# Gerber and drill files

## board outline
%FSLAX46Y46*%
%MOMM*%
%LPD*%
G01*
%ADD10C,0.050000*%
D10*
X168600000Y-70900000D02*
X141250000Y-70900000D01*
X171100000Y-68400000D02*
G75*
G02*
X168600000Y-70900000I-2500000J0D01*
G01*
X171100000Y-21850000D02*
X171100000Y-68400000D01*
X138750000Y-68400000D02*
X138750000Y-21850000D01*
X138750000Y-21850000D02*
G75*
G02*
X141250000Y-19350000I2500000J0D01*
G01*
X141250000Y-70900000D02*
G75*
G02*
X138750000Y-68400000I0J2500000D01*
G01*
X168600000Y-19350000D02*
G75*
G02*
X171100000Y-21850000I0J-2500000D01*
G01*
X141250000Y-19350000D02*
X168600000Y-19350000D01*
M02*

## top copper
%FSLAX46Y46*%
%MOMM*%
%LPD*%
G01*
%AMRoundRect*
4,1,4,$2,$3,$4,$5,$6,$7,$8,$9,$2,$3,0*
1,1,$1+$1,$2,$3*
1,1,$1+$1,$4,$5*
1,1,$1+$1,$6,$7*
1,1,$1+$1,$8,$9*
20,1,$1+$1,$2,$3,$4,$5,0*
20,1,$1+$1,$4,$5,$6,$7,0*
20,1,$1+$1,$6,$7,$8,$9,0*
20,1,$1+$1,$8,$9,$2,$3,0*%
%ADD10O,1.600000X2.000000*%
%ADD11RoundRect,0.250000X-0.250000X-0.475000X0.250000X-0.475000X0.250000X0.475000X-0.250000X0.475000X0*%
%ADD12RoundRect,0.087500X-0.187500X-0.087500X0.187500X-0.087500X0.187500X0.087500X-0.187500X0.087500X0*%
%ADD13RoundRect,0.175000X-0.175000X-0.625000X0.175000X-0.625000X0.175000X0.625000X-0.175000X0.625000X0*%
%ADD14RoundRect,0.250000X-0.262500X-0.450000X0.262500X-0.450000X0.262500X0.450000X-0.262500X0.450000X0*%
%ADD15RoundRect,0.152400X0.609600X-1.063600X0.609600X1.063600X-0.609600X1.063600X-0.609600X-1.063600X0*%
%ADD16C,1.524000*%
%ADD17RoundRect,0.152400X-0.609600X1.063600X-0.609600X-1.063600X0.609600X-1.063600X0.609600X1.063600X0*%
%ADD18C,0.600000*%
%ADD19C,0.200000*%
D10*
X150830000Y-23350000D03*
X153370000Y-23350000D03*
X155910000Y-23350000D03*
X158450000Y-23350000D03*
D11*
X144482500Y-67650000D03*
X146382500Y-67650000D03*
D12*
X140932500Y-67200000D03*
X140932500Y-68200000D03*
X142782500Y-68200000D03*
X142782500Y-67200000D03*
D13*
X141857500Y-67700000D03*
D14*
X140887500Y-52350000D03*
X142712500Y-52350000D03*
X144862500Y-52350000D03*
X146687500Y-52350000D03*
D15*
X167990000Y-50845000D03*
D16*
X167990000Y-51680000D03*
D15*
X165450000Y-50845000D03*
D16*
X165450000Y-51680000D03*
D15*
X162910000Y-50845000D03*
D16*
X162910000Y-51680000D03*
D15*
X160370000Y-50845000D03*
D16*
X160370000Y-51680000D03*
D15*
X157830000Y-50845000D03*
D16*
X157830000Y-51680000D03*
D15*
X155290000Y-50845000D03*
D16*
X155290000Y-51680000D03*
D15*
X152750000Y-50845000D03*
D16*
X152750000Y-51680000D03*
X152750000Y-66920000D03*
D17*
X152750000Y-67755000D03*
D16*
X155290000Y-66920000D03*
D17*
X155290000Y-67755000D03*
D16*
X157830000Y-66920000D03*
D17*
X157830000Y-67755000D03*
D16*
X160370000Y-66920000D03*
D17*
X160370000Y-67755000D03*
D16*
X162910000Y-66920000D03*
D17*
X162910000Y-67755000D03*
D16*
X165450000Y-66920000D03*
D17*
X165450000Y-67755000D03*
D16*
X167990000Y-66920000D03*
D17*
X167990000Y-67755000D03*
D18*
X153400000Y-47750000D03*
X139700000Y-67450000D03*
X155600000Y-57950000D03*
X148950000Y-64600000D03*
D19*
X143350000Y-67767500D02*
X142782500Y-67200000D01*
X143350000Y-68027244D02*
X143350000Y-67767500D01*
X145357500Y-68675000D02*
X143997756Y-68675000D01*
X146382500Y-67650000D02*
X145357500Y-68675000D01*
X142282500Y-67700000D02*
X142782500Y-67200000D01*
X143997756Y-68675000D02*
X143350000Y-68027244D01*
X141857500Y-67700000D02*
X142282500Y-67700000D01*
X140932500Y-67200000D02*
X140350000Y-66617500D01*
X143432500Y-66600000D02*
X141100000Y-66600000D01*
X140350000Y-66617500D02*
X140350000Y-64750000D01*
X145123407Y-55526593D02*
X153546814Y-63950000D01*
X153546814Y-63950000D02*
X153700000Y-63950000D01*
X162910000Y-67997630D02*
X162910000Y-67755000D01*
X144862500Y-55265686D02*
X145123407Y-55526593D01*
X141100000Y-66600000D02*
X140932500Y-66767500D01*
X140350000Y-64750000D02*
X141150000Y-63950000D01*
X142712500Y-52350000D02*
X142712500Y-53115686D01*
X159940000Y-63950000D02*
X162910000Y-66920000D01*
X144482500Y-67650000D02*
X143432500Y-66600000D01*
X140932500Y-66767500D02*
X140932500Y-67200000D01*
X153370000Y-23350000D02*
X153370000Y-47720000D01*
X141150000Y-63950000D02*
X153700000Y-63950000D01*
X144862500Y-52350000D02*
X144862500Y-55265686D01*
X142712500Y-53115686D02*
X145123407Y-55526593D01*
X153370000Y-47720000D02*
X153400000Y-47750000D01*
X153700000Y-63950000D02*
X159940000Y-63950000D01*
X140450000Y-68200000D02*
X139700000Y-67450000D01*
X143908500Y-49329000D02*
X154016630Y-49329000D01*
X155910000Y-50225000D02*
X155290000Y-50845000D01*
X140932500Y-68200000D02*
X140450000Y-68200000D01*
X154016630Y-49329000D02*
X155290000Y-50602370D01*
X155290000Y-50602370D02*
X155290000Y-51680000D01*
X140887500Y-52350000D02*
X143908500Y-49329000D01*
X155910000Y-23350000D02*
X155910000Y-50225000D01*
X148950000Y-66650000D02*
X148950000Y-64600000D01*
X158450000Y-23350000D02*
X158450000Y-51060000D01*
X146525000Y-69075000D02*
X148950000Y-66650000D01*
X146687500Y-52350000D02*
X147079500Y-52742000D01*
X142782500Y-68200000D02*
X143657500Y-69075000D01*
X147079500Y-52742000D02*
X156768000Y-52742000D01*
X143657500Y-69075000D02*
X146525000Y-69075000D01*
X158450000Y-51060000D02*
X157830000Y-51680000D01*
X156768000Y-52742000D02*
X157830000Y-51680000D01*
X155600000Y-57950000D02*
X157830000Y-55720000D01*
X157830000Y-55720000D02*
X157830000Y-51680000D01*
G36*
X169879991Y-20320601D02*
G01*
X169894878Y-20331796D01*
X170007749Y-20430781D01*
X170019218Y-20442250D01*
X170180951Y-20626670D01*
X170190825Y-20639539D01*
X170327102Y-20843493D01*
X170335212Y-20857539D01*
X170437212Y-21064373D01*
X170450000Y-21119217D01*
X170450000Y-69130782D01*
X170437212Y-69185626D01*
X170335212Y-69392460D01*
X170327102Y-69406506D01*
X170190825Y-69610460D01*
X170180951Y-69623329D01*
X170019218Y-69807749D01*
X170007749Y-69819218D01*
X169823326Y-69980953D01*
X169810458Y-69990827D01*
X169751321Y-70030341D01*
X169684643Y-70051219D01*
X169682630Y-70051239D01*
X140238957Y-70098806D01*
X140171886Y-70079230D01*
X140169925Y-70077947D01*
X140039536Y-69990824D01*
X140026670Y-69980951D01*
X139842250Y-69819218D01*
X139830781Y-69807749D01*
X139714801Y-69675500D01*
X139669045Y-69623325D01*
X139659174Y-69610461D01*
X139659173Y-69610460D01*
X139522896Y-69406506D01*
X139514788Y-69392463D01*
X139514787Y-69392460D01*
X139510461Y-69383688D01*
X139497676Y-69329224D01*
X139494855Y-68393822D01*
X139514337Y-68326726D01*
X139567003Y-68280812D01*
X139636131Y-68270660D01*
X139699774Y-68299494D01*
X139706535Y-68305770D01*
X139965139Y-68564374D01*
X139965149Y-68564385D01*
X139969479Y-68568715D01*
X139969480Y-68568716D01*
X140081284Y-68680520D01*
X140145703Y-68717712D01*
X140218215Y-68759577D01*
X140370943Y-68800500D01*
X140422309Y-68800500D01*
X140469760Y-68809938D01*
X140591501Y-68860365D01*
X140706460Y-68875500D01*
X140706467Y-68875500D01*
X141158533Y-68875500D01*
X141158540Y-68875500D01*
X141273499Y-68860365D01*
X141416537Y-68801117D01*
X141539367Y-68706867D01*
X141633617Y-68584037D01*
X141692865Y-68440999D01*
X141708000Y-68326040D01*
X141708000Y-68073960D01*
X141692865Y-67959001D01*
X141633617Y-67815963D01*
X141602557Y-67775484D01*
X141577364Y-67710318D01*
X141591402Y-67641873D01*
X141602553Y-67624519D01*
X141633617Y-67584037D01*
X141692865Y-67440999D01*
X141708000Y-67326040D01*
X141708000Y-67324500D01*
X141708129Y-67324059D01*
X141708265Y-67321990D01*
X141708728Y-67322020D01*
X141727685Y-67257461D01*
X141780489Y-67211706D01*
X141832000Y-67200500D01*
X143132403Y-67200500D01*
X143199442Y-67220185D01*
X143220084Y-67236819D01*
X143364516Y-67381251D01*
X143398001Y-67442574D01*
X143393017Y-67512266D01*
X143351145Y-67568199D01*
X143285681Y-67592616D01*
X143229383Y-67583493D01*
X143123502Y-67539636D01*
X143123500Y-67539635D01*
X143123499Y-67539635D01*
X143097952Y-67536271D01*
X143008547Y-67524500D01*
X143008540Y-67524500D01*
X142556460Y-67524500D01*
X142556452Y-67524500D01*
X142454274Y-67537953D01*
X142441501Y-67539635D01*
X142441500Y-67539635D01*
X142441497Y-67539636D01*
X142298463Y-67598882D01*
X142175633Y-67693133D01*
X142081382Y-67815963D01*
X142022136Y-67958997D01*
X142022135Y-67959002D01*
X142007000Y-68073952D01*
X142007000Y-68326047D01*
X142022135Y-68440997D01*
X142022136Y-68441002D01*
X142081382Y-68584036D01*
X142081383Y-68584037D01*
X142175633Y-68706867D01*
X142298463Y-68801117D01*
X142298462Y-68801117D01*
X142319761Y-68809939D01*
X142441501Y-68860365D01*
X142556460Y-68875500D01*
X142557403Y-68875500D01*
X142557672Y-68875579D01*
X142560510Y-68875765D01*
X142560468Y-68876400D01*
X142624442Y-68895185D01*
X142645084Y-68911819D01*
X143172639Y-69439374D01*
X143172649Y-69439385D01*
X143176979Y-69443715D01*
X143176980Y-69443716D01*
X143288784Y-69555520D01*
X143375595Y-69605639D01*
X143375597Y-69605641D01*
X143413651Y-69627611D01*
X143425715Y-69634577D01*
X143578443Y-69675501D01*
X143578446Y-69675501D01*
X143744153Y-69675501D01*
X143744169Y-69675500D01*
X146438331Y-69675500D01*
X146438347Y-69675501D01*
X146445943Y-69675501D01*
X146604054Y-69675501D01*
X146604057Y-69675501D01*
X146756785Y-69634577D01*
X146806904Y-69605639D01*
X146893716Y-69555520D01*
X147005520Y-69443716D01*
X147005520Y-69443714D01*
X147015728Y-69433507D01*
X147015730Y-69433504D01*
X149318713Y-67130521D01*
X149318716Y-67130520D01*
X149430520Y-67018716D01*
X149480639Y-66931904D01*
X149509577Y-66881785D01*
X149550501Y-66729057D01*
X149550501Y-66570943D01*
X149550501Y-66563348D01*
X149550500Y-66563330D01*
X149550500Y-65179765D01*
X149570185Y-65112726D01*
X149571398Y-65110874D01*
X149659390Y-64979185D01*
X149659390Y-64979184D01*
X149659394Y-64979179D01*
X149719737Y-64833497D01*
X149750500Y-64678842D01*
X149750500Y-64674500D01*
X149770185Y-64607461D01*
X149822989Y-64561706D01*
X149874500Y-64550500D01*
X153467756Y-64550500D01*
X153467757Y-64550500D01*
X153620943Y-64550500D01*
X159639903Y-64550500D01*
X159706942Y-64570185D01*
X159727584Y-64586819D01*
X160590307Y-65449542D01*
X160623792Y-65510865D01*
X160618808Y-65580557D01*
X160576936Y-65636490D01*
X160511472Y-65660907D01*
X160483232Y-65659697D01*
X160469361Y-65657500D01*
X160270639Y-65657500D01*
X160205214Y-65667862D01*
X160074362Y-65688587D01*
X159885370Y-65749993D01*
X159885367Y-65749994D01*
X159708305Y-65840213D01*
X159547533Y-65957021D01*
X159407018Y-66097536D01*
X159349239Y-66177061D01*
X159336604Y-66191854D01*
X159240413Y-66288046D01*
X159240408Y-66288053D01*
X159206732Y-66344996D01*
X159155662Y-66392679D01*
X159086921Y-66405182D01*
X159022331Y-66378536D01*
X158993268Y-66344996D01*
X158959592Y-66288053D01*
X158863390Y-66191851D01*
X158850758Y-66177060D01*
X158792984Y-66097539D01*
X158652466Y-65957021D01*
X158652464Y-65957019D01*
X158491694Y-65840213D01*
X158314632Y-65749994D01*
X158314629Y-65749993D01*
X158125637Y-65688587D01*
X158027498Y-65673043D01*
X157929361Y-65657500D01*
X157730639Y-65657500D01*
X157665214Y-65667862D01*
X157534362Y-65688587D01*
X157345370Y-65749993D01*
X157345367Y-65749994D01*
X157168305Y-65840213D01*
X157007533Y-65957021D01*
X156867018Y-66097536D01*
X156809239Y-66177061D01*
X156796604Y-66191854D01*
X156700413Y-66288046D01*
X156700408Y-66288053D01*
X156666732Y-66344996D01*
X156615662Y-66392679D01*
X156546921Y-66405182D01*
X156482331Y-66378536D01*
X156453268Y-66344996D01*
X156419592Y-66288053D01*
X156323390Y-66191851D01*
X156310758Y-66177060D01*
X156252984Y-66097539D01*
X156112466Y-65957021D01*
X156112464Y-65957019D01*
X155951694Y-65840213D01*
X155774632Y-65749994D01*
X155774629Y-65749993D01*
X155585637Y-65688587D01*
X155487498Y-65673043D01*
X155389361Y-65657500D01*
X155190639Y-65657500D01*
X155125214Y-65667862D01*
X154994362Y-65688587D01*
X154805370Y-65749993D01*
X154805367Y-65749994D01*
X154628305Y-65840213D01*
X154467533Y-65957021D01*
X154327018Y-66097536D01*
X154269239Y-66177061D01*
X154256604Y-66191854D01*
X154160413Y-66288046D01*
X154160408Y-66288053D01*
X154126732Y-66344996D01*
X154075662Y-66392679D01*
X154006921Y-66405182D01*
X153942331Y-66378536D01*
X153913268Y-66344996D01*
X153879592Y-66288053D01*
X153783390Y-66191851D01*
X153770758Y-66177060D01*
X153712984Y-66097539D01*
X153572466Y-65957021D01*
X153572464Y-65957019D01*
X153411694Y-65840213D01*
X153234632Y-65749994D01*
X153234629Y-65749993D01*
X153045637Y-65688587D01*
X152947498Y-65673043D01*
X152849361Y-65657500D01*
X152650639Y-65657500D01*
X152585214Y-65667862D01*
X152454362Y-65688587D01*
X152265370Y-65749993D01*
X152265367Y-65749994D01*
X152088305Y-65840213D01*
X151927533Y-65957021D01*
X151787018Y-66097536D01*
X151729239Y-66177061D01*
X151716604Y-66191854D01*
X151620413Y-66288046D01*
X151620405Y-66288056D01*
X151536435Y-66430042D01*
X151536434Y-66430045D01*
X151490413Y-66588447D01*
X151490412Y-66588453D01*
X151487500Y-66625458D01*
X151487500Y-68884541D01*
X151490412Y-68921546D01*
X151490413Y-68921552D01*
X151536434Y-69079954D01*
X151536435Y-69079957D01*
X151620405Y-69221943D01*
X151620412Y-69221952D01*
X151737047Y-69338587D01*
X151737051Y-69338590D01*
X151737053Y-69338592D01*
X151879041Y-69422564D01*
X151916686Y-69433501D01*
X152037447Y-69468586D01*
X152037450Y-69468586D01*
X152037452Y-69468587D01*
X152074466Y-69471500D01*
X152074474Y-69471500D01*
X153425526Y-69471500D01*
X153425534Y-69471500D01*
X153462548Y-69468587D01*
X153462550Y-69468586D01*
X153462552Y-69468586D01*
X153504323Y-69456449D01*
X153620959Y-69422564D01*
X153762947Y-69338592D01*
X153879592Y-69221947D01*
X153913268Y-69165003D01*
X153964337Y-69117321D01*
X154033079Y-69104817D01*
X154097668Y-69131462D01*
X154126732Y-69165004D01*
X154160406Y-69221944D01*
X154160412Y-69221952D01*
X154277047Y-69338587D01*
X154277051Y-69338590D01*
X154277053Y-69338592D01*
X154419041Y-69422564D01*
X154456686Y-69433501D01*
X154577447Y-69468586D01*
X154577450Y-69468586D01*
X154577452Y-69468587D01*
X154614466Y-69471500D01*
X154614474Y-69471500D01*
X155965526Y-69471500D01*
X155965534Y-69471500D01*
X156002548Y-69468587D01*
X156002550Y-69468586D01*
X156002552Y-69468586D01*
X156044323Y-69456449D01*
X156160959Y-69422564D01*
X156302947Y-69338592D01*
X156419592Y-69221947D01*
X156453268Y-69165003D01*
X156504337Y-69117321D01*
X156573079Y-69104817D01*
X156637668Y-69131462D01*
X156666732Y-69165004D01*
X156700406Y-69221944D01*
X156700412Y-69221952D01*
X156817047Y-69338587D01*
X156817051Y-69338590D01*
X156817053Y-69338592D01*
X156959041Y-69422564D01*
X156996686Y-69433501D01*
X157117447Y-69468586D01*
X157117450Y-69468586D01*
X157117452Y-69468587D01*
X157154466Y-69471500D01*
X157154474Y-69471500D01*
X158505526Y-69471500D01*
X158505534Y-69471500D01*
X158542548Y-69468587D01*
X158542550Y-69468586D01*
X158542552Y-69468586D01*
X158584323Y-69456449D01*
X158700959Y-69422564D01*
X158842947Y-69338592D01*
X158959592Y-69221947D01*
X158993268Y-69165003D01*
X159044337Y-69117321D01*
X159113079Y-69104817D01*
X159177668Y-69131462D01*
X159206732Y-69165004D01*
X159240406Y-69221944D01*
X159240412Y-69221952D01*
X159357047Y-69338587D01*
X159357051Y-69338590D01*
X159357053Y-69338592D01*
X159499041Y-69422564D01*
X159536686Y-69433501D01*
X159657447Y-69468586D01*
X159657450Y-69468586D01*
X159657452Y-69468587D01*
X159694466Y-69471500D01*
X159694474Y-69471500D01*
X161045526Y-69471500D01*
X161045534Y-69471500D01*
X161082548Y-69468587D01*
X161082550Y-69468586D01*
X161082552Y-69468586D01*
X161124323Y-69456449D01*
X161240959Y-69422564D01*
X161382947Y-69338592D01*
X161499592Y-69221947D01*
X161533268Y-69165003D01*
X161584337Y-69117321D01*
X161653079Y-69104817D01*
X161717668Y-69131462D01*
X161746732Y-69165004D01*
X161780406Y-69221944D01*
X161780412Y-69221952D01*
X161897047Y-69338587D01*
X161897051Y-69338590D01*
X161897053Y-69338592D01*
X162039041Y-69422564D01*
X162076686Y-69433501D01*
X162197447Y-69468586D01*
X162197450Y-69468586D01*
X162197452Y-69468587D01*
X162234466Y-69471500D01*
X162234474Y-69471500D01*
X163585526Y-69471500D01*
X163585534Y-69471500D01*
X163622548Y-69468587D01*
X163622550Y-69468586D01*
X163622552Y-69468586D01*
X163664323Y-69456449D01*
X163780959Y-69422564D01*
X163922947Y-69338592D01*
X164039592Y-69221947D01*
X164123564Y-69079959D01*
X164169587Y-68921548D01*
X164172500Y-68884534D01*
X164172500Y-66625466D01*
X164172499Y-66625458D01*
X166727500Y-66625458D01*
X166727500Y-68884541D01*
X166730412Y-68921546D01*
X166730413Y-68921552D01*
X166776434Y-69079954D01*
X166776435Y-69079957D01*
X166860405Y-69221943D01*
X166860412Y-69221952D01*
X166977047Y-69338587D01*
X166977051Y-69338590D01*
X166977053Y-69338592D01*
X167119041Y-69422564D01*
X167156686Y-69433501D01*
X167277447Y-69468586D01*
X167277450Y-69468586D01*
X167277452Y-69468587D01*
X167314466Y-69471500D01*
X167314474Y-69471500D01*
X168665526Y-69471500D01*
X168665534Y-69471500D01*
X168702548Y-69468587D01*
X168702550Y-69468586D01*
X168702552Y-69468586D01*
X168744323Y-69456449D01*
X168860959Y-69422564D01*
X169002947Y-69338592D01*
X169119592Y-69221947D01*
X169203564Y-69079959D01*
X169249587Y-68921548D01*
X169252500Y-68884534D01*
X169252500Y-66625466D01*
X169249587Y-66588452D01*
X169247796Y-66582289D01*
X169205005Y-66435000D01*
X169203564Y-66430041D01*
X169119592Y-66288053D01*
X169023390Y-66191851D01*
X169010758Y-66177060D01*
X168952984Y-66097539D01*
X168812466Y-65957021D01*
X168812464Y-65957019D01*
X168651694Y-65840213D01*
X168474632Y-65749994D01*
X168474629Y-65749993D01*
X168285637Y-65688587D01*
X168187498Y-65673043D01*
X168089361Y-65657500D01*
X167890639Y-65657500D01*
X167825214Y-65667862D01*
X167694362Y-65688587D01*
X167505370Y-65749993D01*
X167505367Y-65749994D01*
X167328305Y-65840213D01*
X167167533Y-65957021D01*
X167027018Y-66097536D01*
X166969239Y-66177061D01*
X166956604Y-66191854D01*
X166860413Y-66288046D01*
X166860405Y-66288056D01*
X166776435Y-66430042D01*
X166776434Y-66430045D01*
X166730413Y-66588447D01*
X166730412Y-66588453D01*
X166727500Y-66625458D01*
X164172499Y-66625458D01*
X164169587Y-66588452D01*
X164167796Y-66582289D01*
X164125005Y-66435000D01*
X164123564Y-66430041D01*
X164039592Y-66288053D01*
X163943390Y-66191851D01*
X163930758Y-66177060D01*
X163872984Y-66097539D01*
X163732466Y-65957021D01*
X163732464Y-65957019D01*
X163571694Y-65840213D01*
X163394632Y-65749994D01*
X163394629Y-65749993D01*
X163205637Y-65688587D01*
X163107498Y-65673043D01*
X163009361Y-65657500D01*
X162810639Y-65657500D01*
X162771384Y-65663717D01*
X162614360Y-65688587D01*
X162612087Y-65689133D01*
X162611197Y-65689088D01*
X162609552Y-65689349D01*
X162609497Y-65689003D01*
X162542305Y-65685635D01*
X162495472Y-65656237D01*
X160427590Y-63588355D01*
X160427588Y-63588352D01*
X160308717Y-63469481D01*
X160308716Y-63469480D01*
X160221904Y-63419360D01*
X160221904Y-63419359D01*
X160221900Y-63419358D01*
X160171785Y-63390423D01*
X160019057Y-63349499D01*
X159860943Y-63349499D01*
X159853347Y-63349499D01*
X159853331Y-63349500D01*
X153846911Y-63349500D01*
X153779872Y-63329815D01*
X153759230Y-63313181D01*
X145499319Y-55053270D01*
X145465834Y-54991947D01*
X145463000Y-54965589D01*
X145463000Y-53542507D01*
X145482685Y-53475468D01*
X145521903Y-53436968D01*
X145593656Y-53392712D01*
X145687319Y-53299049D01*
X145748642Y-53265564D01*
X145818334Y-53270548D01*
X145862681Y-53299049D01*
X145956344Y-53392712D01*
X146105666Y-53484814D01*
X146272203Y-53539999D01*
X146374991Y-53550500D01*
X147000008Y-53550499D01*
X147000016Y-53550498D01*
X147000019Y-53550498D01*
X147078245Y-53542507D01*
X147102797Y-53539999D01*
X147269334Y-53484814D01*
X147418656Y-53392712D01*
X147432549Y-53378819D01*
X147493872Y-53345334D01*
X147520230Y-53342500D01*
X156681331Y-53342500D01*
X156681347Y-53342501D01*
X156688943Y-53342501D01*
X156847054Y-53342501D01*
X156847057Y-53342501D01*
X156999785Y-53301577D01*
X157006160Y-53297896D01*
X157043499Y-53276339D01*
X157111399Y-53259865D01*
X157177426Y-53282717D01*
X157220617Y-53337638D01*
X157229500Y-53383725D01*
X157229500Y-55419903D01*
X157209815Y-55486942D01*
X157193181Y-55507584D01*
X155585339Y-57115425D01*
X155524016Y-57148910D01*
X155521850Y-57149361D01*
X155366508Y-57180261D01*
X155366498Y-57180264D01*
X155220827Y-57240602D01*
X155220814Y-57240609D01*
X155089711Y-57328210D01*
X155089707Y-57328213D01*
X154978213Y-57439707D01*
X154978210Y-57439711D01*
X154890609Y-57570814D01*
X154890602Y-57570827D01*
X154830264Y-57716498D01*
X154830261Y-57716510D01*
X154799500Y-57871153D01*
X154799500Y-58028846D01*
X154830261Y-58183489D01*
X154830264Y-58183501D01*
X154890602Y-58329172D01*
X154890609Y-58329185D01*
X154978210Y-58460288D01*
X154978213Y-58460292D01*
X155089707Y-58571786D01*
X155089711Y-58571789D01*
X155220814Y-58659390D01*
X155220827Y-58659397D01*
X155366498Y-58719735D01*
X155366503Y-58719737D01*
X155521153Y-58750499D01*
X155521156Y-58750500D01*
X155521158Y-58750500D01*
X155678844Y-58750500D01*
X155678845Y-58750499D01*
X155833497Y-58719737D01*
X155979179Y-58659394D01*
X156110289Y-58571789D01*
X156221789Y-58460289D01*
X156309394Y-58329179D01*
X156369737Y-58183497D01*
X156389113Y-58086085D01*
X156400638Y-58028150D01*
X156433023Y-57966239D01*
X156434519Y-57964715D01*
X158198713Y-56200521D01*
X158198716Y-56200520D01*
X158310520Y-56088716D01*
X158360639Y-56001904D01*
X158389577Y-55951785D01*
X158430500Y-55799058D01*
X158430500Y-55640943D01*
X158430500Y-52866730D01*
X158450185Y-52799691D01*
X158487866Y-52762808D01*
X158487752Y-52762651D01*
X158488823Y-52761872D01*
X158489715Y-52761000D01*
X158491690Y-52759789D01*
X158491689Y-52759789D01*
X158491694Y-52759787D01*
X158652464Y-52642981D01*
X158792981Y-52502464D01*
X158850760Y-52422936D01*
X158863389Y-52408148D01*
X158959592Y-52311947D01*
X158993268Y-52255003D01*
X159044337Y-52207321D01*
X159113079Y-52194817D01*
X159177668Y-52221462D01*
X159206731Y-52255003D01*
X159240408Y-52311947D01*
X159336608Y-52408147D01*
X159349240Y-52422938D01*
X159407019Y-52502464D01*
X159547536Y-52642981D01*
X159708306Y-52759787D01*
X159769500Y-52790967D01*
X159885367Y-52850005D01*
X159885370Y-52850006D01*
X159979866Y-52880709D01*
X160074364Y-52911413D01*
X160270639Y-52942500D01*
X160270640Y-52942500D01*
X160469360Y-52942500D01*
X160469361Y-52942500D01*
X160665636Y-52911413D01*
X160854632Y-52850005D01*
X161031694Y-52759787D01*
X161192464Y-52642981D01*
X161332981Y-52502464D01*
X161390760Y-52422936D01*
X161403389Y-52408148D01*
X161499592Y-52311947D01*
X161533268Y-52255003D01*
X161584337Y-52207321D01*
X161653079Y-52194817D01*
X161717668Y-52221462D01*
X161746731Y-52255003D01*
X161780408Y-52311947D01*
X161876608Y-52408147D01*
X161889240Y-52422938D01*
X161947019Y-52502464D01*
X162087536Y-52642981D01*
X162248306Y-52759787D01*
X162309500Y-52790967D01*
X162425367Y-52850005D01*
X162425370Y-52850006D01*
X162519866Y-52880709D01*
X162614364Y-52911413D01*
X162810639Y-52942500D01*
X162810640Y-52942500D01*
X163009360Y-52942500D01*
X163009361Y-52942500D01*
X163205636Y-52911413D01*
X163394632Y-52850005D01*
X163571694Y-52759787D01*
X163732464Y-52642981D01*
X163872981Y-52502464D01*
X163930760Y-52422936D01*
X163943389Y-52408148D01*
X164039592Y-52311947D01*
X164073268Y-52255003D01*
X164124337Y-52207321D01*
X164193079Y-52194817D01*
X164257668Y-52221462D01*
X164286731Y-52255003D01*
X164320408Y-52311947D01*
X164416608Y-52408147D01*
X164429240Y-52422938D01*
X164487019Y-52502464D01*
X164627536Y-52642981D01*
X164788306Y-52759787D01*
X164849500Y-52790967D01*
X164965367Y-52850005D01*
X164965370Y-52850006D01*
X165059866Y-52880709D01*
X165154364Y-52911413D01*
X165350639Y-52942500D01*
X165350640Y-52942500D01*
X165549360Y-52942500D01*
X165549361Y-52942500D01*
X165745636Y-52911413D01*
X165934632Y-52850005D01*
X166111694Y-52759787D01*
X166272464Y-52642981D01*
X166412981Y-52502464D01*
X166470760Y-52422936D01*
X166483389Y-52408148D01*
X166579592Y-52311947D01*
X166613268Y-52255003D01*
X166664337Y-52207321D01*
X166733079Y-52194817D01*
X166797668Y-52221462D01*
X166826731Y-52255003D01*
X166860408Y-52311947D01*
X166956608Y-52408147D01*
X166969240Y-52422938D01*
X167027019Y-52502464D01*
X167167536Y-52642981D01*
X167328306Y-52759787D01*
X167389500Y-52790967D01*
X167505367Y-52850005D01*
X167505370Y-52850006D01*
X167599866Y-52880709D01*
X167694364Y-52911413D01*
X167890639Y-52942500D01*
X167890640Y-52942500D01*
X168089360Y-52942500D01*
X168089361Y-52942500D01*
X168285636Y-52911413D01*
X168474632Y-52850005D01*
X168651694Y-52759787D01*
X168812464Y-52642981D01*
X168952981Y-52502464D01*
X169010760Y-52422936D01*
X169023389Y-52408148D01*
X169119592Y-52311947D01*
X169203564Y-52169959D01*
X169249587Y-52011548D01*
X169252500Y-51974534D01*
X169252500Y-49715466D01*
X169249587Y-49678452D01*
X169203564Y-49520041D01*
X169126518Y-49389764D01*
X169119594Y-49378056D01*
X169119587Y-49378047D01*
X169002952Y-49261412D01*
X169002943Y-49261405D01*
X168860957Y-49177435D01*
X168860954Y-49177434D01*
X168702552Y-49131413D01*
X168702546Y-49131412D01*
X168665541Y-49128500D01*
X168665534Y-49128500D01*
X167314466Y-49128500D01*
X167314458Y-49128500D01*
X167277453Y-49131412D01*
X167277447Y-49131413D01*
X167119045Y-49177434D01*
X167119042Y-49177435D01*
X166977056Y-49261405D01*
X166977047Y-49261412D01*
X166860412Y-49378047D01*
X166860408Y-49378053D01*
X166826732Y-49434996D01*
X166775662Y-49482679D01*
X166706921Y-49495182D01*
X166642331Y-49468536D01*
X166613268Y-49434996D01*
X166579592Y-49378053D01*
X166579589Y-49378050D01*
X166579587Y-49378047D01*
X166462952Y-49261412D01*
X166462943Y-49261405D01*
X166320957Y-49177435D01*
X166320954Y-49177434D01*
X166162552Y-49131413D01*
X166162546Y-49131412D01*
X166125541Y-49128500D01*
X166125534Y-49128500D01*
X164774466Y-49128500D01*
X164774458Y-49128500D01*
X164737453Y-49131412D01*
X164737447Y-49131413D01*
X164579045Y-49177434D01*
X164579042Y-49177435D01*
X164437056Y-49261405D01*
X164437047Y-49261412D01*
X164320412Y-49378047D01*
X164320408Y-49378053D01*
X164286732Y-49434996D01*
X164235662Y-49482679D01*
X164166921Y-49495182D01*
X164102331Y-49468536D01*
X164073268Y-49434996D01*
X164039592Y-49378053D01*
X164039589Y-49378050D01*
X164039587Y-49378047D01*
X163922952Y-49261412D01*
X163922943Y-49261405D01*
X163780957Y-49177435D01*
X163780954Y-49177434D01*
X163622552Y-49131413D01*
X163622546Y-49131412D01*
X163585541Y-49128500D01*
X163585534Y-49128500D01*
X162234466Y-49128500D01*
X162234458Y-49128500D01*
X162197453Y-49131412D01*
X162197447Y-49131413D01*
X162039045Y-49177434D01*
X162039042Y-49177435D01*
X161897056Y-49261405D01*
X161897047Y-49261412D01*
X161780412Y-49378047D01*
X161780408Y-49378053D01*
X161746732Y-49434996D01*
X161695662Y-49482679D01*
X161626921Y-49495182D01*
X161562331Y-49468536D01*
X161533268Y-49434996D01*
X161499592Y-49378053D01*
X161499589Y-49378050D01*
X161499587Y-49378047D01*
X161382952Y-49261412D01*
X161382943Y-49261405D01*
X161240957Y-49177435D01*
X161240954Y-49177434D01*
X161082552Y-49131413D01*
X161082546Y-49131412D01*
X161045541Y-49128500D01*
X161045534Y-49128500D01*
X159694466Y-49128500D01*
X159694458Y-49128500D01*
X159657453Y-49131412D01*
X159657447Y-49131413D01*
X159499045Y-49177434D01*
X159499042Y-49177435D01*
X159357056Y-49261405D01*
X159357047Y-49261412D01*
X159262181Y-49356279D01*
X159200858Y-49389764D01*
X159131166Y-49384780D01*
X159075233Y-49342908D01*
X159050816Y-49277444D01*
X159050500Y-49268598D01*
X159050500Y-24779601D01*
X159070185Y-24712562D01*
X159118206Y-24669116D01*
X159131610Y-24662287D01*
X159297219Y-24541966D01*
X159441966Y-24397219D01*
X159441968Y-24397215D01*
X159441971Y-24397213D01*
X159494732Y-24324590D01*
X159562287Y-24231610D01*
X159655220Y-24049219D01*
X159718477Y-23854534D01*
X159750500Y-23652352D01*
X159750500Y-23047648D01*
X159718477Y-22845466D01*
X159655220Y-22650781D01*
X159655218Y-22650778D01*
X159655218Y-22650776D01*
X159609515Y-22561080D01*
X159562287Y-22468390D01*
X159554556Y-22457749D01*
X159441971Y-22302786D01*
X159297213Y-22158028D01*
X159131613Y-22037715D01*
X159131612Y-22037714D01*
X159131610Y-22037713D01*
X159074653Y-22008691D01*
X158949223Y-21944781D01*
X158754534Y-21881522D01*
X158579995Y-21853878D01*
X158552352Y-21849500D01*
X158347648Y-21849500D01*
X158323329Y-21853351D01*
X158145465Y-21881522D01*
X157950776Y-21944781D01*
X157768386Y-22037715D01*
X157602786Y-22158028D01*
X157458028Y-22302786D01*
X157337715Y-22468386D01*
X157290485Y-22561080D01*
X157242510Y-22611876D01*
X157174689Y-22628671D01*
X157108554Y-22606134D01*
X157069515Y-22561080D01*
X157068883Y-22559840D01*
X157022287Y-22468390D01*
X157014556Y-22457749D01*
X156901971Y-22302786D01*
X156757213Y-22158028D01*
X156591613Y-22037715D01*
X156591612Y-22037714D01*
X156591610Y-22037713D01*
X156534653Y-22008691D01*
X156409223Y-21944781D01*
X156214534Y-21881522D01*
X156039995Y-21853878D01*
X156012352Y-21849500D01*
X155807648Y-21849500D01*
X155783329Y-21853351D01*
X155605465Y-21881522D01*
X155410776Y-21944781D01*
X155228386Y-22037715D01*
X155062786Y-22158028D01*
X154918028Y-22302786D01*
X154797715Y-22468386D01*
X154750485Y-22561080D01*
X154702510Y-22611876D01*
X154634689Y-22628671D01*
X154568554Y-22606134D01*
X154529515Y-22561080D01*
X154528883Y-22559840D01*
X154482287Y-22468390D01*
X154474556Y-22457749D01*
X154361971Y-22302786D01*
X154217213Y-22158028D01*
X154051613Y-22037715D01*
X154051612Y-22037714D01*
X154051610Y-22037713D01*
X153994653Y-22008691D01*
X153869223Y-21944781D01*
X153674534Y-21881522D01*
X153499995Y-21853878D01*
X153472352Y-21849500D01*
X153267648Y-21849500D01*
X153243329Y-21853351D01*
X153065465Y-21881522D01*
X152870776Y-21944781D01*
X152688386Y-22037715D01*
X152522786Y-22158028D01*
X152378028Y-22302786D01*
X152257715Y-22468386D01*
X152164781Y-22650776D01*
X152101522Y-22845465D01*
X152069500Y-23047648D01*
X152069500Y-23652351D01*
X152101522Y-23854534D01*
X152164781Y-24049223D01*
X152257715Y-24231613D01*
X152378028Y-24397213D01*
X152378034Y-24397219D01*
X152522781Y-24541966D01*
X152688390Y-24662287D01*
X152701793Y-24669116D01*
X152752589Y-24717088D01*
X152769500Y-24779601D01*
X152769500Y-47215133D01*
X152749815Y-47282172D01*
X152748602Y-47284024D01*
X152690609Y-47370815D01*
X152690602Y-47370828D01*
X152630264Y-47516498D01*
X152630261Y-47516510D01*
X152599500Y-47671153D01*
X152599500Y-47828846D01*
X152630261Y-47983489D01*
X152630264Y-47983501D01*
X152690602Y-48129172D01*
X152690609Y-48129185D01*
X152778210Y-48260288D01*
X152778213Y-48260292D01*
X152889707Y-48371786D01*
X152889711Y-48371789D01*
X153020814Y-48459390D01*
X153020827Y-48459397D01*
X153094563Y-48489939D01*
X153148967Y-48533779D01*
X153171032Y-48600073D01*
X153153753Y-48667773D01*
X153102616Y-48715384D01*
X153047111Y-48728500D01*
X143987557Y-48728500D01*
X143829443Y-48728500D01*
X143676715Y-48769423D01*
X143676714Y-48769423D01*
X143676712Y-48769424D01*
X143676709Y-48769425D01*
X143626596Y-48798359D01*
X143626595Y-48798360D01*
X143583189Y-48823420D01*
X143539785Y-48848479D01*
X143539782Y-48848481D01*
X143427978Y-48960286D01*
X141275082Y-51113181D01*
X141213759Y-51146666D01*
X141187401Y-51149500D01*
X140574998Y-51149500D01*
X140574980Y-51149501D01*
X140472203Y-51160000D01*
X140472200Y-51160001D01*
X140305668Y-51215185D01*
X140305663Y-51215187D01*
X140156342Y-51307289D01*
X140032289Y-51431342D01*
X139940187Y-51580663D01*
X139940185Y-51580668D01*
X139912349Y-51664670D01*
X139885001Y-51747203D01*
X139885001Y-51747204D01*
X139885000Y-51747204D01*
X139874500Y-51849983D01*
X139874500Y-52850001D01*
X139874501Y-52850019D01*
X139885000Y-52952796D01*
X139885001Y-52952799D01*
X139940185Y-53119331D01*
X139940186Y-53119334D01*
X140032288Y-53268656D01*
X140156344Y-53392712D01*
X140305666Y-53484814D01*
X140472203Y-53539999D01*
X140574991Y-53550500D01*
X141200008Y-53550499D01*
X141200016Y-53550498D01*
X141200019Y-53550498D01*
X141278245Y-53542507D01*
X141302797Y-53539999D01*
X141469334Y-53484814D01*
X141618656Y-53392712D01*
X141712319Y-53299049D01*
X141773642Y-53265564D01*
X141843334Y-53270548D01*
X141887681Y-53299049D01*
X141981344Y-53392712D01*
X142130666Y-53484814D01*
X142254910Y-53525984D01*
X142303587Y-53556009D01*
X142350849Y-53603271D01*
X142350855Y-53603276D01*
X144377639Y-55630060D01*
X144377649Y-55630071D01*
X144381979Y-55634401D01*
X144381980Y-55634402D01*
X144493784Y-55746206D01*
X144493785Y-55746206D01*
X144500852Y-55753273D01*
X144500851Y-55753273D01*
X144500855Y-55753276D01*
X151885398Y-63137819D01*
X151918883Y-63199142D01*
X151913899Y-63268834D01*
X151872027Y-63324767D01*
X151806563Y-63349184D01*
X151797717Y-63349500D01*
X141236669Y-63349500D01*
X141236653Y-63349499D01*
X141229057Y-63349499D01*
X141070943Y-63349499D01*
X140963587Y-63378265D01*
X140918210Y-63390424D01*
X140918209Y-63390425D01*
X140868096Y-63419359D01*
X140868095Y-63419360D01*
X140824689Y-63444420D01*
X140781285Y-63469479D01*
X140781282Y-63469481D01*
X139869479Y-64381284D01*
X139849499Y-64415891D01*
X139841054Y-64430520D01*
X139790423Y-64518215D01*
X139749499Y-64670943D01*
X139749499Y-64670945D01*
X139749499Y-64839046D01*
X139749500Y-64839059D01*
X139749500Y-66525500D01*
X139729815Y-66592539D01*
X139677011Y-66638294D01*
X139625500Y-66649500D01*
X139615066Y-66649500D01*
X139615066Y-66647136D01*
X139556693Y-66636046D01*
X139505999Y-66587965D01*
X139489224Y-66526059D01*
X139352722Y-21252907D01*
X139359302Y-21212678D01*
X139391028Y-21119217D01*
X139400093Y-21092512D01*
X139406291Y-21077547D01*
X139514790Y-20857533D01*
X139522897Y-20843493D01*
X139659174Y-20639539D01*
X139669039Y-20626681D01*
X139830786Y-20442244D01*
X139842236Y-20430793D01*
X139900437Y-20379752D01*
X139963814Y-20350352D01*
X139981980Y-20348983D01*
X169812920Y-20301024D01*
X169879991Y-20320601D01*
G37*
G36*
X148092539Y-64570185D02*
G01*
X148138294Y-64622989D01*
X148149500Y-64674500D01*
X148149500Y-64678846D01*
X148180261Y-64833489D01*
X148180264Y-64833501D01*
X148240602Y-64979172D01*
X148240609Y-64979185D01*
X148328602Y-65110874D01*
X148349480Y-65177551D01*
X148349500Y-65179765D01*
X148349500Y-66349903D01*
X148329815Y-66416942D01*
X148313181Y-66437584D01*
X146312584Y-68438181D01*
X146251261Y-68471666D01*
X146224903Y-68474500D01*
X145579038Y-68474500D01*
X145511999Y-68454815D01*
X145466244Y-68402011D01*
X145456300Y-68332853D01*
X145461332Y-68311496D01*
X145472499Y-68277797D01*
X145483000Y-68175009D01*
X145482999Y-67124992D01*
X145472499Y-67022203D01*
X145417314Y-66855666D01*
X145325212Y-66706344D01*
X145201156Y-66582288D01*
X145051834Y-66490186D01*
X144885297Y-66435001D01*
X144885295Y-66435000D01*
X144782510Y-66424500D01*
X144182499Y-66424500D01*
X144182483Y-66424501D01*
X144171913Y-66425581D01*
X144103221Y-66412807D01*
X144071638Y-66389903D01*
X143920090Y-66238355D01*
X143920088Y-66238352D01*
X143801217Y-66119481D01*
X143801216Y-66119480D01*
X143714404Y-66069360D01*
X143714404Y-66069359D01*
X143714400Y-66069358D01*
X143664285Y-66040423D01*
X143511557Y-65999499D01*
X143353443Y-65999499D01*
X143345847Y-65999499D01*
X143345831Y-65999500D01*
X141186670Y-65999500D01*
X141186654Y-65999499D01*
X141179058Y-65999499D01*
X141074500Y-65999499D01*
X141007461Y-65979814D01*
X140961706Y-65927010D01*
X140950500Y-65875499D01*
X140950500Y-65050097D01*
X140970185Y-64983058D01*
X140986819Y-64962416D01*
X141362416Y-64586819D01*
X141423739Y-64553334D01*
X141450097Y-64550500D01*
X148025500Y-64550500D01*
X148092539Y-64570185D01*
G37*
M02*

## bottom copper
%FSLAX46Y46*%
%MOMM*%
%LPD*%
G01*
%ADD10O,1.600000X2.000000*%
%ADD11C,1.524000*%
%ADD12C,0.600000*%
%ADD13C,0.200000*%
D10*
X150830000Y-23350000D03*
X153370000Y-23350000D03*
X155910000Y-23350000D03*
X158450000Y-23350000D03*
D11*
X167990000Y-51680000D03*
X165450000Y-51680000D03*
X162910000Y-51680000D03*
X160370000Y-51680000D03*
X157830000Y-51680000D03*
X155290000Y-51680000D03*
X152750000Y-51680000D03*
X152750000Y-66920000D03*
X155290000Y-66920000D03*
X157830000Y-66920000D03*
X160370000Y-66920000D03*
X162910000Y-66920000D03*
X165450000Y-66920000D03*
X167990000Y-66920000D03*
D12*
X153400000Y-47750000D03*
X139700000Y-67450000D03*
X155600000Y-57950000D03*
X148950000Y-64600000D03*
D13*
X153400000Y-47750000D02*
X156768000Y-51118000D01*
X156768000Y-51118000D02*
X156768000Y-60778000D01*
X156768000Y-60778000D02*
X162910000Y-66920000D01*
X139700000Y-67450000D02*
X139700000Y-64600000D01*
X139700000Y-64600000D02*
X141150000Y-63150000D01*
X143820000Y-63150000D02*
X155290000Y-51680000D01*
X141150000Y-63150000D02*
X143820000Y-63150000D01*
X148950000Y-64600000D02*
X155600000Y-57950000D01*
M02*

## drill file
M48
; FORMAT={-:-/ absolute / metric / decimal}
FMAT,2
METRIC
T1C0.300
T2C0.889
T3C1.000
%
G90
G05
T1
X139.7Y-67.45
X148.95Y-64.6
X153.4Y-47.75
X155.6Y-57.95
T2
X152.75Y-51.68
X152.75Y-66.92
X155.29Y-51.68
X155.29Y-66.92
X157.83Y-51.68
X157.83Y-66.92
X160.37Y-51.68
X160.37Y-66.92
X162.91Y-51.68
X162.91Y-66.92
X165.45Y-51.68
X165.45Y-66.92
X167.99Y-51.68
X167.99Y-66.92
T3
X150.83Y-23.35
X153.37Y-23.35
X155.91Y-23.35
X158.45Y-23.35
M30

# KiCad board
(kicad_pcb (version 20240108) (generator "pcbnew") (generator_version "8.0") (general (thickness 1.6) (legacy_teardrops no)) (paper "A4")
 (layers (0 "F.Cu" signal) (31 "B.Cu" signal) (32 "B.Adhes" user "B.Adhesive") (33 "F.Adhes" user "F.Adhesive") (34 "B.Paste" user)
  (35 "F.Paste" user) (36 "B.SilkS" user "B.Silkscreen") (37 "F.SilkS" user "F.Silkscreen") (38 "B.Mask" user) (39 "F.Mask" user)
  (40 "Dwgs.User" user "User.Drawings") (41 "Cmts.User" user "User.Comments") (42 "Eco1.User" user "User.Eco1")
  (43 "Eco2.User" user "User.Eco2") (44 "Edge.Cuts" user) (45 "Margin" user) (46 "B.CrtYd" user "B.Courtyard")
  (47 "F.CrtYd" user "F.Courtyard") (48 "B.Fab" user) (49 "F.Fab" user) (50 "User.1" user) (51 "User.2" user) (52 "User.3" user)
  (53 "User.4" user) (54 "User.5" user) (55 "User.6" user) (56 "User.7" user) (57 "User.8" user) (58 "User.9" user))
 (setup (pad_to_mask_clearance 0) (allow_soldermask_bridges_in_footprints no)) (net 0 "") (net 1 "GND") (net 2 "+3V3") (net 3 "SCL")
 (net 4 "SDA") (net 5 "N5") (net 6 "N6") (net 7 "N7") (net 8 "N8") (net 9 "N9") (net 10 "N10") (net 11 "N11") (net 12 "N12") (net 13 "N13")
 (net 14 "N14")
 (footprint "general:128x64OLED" (layer "F.Cu") (at 154.45 33.95)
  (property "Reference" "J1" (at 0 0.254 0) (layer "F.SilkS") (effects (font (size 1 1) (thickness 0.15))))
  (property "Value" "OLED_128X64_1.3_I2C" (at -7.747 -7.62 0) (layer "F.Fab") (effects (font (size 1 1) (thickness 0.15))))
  (pad "1" thru_hole oval (at -3.62 -10.6 90) (size 2 1.6) (drill 1) (layers "*.Cu" "*.Mask") (remove_unused_layers no) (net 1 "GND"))
  (pad "2" thru_hole oval (at -1.08 -10.6 90) (size 2 1.6) (drill 1) (layers "*.Cu" "*.Mask") (remove_unused_layers no) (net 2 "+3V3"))
  (pad "3" thru_hole oval (at 1.46 -10.6 90) (size 2 1.6) (drill 1) (layers "*.Cu" "*.Mask") (remove_unused_layers no) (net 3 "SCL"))
  (pad "4" thru_hole oval (at 4 -10.6 90) (size 2 1.6) (drill 1) (layers "*.Cu" "*.Mask") (remove_unused_layers no) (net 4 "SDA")))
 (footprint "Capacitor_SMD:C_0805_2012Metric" (layer "F.Cu") (at 145.4325 67.65)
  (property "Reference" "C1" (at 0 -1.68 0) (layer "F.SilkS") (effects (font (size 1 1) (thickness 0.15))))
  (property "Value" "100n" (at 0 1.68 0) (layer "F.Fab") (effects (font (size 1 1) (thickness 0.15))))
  (pad "1" smd roundrect (at -0.95 0) (size 1 1.45) (layers "F.Cu" "F.Paste" "F.Mask") (roundrect_rratio 0.25) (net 2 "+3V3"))
  (pad "2" smd roundrect (at 0.95 0) (size 1 1.45) (layers "F.Cu" "F.Paste" "F.Mask") (roundrect_rratio 0.25) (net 1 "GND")))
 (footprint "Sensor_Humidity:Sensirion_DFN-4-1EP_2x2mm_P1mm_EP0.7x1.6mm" (layer "F.Cu") (at 141.8575 67.7)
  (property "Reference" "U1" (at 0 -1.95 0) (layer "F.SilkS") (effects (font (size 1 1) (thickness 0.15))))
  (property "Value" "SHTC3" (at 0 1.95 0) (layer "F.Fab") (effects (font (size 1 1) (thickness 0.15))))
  (pad "" smd roundrect (at -1.025 -0.5) (size 0.55 0.35) (layers "F.Paste") (roundrect_rratio 0.25))
  (pad "" smd roundrect (at -1.025 0.5) (size 0.55 0.35) (layers "F.Paste") (roundrect_rratio 0.25))
  (pad "" smd roundrect (at 0 0) (size 0.5 1.4) (layers "F.Paste") (roundrect_rratio 0.25))
  (pad "" smd roundrect (at 1.025 -0.5 180) (size 0.55 0.35) (layers "F.Paste") (roundrect_rratio 0.25))
  (pad "" smd roundrect (at 1.025 0.5 180) (size 0.55 0.35) (layers "F.Paste") (roundrect_rratio 0.25))
  (pad "1" smd roundrect (at -0.925 -0.5) (size 0.55 0.35) (layers "F.Cu" "F.Mask") (roundrect_rratio 0.25) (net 2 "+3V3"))
  (pad "2" smd roundrect (at -0.925 0.5) (size 0.55 0.35) (layers "F.Cu" "F.Mask") (roundrect_rratio 0.25) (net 3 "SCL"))
  (pad "3" smd roundrect (at 0.925 0.5) (size 0.55 0.35) (layers "F.Cu" "F.Mask") (roundrect_rratio 0.25) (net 4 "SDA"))
  (pad "4" smd roundrect (at 0.925 -0.5) (size 0.55 0.35) (layers "F.Cu" "F.Mask") (roundrect_rratio 0.25) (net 1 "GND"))
  (pad "5" smd roundrect (at 0 0) (size 0.7 1.6) (layers "F.Cu" "F.Mask") (roundrect_rratio 0.25) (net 1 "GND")))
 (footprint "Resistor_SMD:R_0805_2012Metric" (layer "F.Cu") (at 141.8 52.35)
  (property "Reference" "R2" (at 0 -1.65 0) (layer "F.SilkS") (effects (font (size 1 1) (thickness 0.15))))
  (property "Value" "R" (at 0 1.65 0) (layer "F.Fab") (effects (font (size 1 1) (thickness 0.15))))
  (pad "1" smd roundrect (at -0.9125 0) (size 1.025 1.4) (layers "F.Cu" "F.Paste" "F.Mask") (roundrect_rratio 0.243902) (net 3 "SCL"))
  (pad "2" smd roundrect (at 0.9125 0) (size 1.025 1.4) (layers "F.Cu" "F.Paste" "F.Mask") (roundrect_rratio 0.243902) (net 2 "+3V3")))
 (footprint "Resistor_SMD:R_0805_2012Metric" (layer "F.Cu") (at 145.775 52.35)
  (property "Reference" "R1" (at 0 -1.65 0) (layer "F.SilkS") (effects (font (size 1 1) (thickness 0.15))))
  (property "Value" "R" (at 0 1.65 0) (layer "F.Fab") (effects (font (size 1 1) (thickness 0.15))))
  (pad "1" smd roundrect (at -0.9125 0) (size 1.025 1.4) (layers "F.Cu" "F.Paste" "F.Mask") (roundrect_rratio 0.243902) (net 2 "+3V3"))
  (pad "2" smd roundrect (at 0.9125 0) (size 1.025 1.4) (layers "F.Cu" "F.Paste" "F.Mask") (roundrect_rratio 0.243902) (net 4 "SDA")))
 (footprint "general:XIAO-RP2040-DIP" (layer "F.Cu") (at 160.37 59.3 -90)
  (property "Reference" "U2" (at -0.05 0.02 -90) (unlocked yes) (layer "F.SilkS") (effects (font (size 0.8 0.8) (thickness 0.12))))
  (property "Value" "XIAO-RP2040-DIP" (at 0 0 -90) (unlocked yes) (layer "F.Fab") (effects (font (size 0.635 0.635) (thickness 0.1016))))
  (pad "1" smd roundrect (at -8.455 -7.62 90) (size 2.432 1.524) (layers "F.Cu" "F.Mask") (roundrect_rratio 0.1) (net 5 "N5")
   (thermal_bridge_angle 45))
  (pad "1" thru_hole circle (at -7.62 -7.62 90) (size 1.524 1.524) (drill 0.889) (layers "*.Cu" "*.Mask") (remove_unused_layers no)
   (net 5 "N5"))
  (pad "2" smd roundrect (at -8.455 -5.08 90) (size 2.432 1.524) (layers "F.Cu" "F.Mask") (roundrect_rratio 0.1) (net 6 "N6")
   (thermal_bridge_angle 45))
  (pad "2" thru_hole circle (at -7.62 -5.08 90) (size 1.524 1.524) (drill 0.889) (layers "*.Cu" "*.Mask") (remove_unused_layers no)
   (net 6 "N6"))
  (pad "3" smd roundrect (at -8.455 -2.54 90) (size 2.432 1.524) (layers "F.Cu" "F.Mask") (roundrect_rratio 0.1) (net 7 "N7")
   (thermal_bridge_angle 45))
  (pad "3" thru_hole circle (at -7.62 -2.54 90) (size 1.524 1.524) (drill 0.889) (layers "*.Cu" "*.Mask") (remove_unused_layers no)
   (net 7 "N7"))
  (pad "4" smd roundrect (at -8.455 0 90) (size 2.432 1.524) (layers "F.Cu" "F.Mask") (roundrect_rratio 0.1) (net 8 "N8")
   (thermal_bridge_angle 45))
  (pad "4" thru_hole circle (at -7.62 0 90) (size 1.524 1.524) (drill 0.889) (layers "*.Cu" "*.Mask") (remove_unused_layers no) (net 8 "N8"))
  (pad "5" smd roundrect (at -8.455 2.54 90) (size 2.432 1.524) (layers "F.Cu" "F.Mask") (roundrect_rratio 0.1) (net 4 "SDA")
   (thermal_bridge_angle 45))
  (pad "5" thru_hole circle (at -7.62 2.54 90) (size 1.524 1.524) (drill 0.889) (layers "*.Cu" "*.Mask") (remove_unused_layers no)
   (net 4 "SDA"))
  (pad "6" smd roundrect (at -8.455 5.08 90) (size 2.432 1.524) (layers "F.Cu" "F.Mask") (roundrect_rratio 0.1) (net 3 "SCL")
   (thermal_bridge_angle 45))
  (pad "6" thru_hole circle (at -7.62 5.08 90) (size 1.524 1.524) (drill 0.889) (layers "*.Cu" "*.Mask") (remove_unused_layers no)
   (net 3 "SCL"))
  (pad "7" smd roundrect (at -8.455 7.62 90) (size 2.432 1.524) (layers "F.Cu" "F.Mask") (roundrect_rratio 0.1) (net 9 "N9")
   (thermal_bridge_angle 45))
  (pad "7" thru_hole circle (at -7.62 7.62 90) (size 1.524 1.524) (drill 0.889) (layers "*.Cu" "*.Mask") (remove_unused_layers no)
   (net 9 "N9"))
  (pad "8" thru_hole circle (at 7.62 7.62 270) (size 1.524 1.524) (drill 0.889) (layers "*.Cu" "*.Mask") (remove_unused_layers no)
   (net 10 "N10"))
  (pad "8" smd roundrect (at 8.455 7.62 270) (size 2.432 1.524) (layers "F.Cu" "F.Mask") (roundrect_rratio 0.1) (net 10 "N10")
   (thermal_bridge_angle 45))
  (pad "9" thru_hole circle (at 7.62 5.08 270) (size 1.524 1.524) (drill 0.889) (layers "*.Cu" "*.Mask") (remove_unused_layers no)
   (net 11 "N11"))
  (pad "9" smd roundrect (at 8.455 5.08 270) (size 2.432 1.524) (layers "F.Cu" "F.Mask") (roundrect_rratio 0.1) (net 11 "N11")
   (thermal_bridge_angle 45))
  (pad "10" thru_hole circle (at 7.62 2.54 270) (size 1.524 1.524) (drill 0.889) (layers "*.Cu" "*.Mask") (remove_unused_layers no)
   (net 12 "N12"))
  (pad "10" smd roundrect (at 8.455 2.54 270) (size 2.432 1.524) (layers "F.Cu" "F.Mask") (roundrect_rratio 0.1) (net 12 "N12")
   (thermal_bridge_angle 45))
  (pad "11" thru_hole circle (at 7.62 0 270) (size 1.524 1.524) (drill 0.889) (layers "*.Cu" "*.Mask") (remove_unused_layers no)
   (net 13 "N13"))
  (pad "11" smd roundrect (at 8.455 0 270) (size 2.432 1.524) (layers "F.Cu" "F.Mask") (roundrect_rratio 0.1) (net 13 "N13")
   (thermal_bridge_angle 45))
  (pad "12" thru_hole circle (at 7.62 -2.54 270) (size 1.524 1.524) (drill 0.889) (layers "*.Cu" "*.Mask") (remove_unused_layers no)
   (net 2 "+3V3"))
  (pad "12" smd roundrect (at 8.455 -2.54 270) (size 2.432 1.524) (layers "F.Cu" "F.Mask") (roundrect_rratio 0.1) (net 2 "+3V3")
   (thermal_bridge_angle 45))
  (pad "13" thru_hole circle (at 7.62 -5.08 270) (size 1.524 1.524) (drill 0.889) (layers "*.Cu" "*.Mask") (remove_unused_layers no)
   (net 1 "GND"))
  (pad "13" smd roundrect (at 8.455 -5.08 270) (size 2.432 1.524) (layers "F.Cu" "F.Mask") (roundrect_rratio 0.1) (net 1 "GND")
   (thermal_bridge_angle 45))
  (pad "14" thru_hole circle (at 7.62 -7.62 270) (size 1.524 1.524) (drill 0.889) (layers "*.Cu" "*.Mask") (remove_unused_layers no)
   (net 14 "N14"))
  (pad "14" smd roundrect (at 8.455 -7.62 270) (size 2.432 1.524) (layers "F.Cu" "F.Mask") (roundrect_rratio 0.1) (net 14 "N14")
   (thermal_bridge_angle 45)))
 (gr_line (start 168.6 70.9) (end 141.25 70.9) (stroke (width 0.05) (type default)) (layer "Edge.Cuts"))
 (gr_arc (start 171.1 68.4) (mid 170.367767 70.167767) (end 168.6 70.9) (stroke (width 0.05) (type default)) (layer "Edge.Cuts"))
 (gr_line (start 171.1 21.85) (end 171.1 68.4) (stroke (width 0.05) (type default)) (layer "Edge.Cuts"))
 (gr_line (start 138.75 68.4) (end 138.75 21.85) (stroke (width 0.05) (type default)) (layer "Edge.Cuts"))
 (gr_arc (start 138.75 21.85) (mid 139.482233 20.082233) (end 141.25 19.35) (stroke (width 0.05) (type default)) (layer "Edge.Cuts"))
 (gr_arc (start 141.25 70.9) (mid 139.482233 70.167767) (end 138.75 68.4) (stroke (width 0.05) (type default)) (layer "Edge.Cuts"))
 (gr_arc (start 168.6 19.35) (mid 170.367767 20.082233) (end 171.1 21.85) (stroke (width 0.05) (type default)) (layer "Edge.Cuts"))
 (gr_line (start 141.25 19.35) (end 168.6 19.35) (stroke (width 0.05) (type default)) (layer "Edge.Cuts"))
 (segment (start 143.35 67.7675) (end 142.7825 67.2) (width 0.2) (layer "F.Cu") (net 1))
 (segment (start 143.35 68.027244) (end 143.35 67.7675) (width 0.2) (layer "F.Cu") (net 1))
 (segment (start 145.3575 68.675) (end 143.997756 68.675) (width 0.2) (layer "F.Cu") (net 1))
 (segment (start 146.3825 67.65) (end 145.3575 68.675) (width 0.2) (layer "F.Cu") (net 1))
 (segment (start 142.2825 67.7) (end 142.7825 67.2) (width 0.2) (layer "F.Cu") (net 1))
 (segment (start 143.997756 68.675) (end 143.35 68.027244) (width 0.2) (layer "F.Cu") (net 1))
 (segment (start 141.8575 67.7) (end 142.2825 67.7) (width 0.2) (layer "F.Cu") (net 1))
 (segment (start 140.9325 67.2) (end 140.35 66.6175) (width 0.2) (layer "F.Cu") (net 2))
 (segment (start 143.4325 66.6) (end 141.1 66.6) (width 0.2) (layer "F.Cu") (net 2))
 (segment (start 140.35 66.6175) (end 140.35 64.75) (width 0.2) (layer "F.Cu") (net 2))
 (segment (start 145.123407 55.526593) (end 153.546814 63.95) (width 0.2) (layer "F.Cu") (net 2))
 (segment (start 153.546814 63.95) (end 153.7 63.95) (width 0.2) (layer "F.Cu") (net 2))
 (segment (start 162.91 67.99763) (end 162.91 67.755) (width 0.2) (layer "F.Cu") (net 2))
 (segment (start 144.8625 55.265686) (end 145.123407 55.526593) (width 0.2) (layer "F.Cu") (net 2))
 (segment (start 141.1 66.6) (end 140.9325 66.7675) (width 0.2) (layer "F.Cu") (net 2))
 (segment (start 140.35 64.75) (end 141.15 63.95) (width 0.2) (layer "F.Cu") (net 2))
 (segment (start 142.7125 52.35) (end 142.7125 53.115686) (width 0.2) (layer "F.Cu") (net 2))
 (segment (start 159.94 63.95) (end 162.91 66.92) (width 0.2) (layer "F.Cu") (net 2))
 (segment (start 144.4825 67.65) (end 143.4325 66.6) (width 0.2) (layer "F.Cu") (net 2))
 (segment (start 140.9325 66.7675) (end 140.9325 67.2) (width 0.2) (layer "F.Cu") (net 2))
 (segment (start 153.37 23.35) (end 153.37 47.72) (width 0.2) (layer "F.Cu") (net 2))
 (segment (start 141.15 63.95) (end 153.7 63.95) (width 0.2) (layer "F.Cu") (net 2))
 (segment (start 144.8625 52.35) (end 144.8625 55.265686) (width 0.2) (layer "F.Cu") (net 2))
 (segment (start 142.7125 53.115686) (end 145.123407 55.526593) (width 0.2) (layer "F.Cu") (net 2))
 (segment (start 153.37 47.72) (end 153.4 47.75) (width 0.2) (layer "F.Cu") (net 2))
 (segment (start 153.7 63.95) (end 159.94 63.95) (width 0.2) (layer "F.Cu") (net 2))
 (via (at 153.4 47.75) (size 0.6) (drill 0.3) (layers "F.Cu" "B.Cu") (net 2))
 (segment (start 153.4 47.75) (end 156.768 51.118) (width 0.2) (layer "B.Cu") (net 2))
 (segment (start 156.768 51.118) (end 156.768 60.778) (width 0.2) (layer "B.Cu") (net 2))
 (segment (start 156.768 60.778) (end 162.91 66.92) (width 0.2) (layer "B.Cu") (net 2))
 (segment (start 140.45 68.2) (end 139.7 67.45) (width 0.2) (layer "F.Cu") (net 3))
 (segment (start 143.9085 49.329) (end 154.01663 49.329) (width 0.2) (layer "F.Cu") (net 3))
 (segment (start 155.91 50.225) (end 155.29 50.845) (width 0.2) (layer "F.Cu") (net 3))
 (segment (start 140.9325 68.2) (end 140.45 68.2) (width 0.2) (layer "F.Cu") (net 3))
 (segment (start 154.01663 49.329) (end 155.29 50.60237) (width 0.2) (layer "F.Cu") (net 3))
 (segment (start 155.29 50.60237) (end 155.29 51.68) (width 0.2) (layer "F.Cu") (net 3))
 (segment (start 140.8875 52.35) (end 143.9085 49.329) (width 0.2) (layer "F.Cu") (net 3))
 (segment (start 155.91 23.35) (end 155.91 50.225) (width 0.2) (layer "F.Cu") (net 3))
 (via (at 139.7 67.45) (size 0.6) (drill 0.3) (layers "F.Cu" "B.Cu") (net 3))
 (segment (start 139.7 67.45) (end 139.7 64.6) (width 0.2) (layer "B.Cu") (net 3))
 (segment (start 139.7 64.6) (end 141.15 63.15) (width 0.2) (layer "B.Cu") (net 3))
 (segment (start 143.82 63.15) (end 155.29 51.68) (width 0.2) (layer "B.Cu") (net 3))
 (segment (start 141.15 63.15) (end 143.82 63.15) (width 0.2) (layer "B.Cu") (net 3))
 (segment (start 148.95 66.65) (end 148.95 64.6) (width 0.2) (layer "F.Cu") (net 4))
 (segment (start 158.45 23.35) (end 158.45 51.06) (width 0.2) (layer "F.Cu") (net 4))
 (segment (start 146.525 69.075) (end 148.95 66.65) (width 0.2) (layer "F.Cu") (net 4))
 (segment (start 146.6875 52.35) (end 147.0795 52.742) (width 0.2) (layer "F.Cu") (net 4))
 (segment (start 142.7825 68.2) (end 143.6575 69.075) (width 0.2) (layer "F.Cu") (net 4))
 (segment (start 147.0795 52.742) (end 156.768 52.742) (width 0.2) (layer "F.Cu") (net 4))
 (segment (start 143.6575 69.075) (end 146.525 69.075) (width 0.2) (layer "F.Cu") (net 4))
 (segment (start 158.45 51.06) (end 157.83 51.68) (width 0.2) (layer "F.Cu") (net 4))
 (segment (start 156.768 52.742) (end 157.83 51.68) (width 0.2) (layer "F.Cu") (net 4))
 (segment (start 155.6 57.95) (end 157.83 55.72) (width 0.2) (layer "F.Cu") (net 4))
 (segment (start 157.83 55.72) (end 157.83 51.68) (width 0.2) (layer "F.Cu") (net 4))
 (via (at 155.6 57.95) (size 0.6) (drill 0.3) (layers "F.Cu" "B.Cu") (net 4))
 (via (at 148.95 64.6) (size 0.6) (drill 0.3) (layers "F.Cu" "B.Cu") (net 4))
 (segment (start 148.95 64.6) (end 155.6 57.95) (width 0.2) (layer "B.Cu") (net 4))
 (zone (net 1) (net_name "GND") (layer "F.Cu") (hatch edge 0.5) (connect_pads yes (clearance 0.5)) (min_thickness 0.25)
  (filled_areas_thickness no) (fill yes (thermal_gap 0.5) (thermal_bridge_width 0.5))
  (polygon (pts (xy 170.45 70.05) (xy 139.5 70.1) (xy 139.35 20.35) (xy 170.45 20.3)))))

